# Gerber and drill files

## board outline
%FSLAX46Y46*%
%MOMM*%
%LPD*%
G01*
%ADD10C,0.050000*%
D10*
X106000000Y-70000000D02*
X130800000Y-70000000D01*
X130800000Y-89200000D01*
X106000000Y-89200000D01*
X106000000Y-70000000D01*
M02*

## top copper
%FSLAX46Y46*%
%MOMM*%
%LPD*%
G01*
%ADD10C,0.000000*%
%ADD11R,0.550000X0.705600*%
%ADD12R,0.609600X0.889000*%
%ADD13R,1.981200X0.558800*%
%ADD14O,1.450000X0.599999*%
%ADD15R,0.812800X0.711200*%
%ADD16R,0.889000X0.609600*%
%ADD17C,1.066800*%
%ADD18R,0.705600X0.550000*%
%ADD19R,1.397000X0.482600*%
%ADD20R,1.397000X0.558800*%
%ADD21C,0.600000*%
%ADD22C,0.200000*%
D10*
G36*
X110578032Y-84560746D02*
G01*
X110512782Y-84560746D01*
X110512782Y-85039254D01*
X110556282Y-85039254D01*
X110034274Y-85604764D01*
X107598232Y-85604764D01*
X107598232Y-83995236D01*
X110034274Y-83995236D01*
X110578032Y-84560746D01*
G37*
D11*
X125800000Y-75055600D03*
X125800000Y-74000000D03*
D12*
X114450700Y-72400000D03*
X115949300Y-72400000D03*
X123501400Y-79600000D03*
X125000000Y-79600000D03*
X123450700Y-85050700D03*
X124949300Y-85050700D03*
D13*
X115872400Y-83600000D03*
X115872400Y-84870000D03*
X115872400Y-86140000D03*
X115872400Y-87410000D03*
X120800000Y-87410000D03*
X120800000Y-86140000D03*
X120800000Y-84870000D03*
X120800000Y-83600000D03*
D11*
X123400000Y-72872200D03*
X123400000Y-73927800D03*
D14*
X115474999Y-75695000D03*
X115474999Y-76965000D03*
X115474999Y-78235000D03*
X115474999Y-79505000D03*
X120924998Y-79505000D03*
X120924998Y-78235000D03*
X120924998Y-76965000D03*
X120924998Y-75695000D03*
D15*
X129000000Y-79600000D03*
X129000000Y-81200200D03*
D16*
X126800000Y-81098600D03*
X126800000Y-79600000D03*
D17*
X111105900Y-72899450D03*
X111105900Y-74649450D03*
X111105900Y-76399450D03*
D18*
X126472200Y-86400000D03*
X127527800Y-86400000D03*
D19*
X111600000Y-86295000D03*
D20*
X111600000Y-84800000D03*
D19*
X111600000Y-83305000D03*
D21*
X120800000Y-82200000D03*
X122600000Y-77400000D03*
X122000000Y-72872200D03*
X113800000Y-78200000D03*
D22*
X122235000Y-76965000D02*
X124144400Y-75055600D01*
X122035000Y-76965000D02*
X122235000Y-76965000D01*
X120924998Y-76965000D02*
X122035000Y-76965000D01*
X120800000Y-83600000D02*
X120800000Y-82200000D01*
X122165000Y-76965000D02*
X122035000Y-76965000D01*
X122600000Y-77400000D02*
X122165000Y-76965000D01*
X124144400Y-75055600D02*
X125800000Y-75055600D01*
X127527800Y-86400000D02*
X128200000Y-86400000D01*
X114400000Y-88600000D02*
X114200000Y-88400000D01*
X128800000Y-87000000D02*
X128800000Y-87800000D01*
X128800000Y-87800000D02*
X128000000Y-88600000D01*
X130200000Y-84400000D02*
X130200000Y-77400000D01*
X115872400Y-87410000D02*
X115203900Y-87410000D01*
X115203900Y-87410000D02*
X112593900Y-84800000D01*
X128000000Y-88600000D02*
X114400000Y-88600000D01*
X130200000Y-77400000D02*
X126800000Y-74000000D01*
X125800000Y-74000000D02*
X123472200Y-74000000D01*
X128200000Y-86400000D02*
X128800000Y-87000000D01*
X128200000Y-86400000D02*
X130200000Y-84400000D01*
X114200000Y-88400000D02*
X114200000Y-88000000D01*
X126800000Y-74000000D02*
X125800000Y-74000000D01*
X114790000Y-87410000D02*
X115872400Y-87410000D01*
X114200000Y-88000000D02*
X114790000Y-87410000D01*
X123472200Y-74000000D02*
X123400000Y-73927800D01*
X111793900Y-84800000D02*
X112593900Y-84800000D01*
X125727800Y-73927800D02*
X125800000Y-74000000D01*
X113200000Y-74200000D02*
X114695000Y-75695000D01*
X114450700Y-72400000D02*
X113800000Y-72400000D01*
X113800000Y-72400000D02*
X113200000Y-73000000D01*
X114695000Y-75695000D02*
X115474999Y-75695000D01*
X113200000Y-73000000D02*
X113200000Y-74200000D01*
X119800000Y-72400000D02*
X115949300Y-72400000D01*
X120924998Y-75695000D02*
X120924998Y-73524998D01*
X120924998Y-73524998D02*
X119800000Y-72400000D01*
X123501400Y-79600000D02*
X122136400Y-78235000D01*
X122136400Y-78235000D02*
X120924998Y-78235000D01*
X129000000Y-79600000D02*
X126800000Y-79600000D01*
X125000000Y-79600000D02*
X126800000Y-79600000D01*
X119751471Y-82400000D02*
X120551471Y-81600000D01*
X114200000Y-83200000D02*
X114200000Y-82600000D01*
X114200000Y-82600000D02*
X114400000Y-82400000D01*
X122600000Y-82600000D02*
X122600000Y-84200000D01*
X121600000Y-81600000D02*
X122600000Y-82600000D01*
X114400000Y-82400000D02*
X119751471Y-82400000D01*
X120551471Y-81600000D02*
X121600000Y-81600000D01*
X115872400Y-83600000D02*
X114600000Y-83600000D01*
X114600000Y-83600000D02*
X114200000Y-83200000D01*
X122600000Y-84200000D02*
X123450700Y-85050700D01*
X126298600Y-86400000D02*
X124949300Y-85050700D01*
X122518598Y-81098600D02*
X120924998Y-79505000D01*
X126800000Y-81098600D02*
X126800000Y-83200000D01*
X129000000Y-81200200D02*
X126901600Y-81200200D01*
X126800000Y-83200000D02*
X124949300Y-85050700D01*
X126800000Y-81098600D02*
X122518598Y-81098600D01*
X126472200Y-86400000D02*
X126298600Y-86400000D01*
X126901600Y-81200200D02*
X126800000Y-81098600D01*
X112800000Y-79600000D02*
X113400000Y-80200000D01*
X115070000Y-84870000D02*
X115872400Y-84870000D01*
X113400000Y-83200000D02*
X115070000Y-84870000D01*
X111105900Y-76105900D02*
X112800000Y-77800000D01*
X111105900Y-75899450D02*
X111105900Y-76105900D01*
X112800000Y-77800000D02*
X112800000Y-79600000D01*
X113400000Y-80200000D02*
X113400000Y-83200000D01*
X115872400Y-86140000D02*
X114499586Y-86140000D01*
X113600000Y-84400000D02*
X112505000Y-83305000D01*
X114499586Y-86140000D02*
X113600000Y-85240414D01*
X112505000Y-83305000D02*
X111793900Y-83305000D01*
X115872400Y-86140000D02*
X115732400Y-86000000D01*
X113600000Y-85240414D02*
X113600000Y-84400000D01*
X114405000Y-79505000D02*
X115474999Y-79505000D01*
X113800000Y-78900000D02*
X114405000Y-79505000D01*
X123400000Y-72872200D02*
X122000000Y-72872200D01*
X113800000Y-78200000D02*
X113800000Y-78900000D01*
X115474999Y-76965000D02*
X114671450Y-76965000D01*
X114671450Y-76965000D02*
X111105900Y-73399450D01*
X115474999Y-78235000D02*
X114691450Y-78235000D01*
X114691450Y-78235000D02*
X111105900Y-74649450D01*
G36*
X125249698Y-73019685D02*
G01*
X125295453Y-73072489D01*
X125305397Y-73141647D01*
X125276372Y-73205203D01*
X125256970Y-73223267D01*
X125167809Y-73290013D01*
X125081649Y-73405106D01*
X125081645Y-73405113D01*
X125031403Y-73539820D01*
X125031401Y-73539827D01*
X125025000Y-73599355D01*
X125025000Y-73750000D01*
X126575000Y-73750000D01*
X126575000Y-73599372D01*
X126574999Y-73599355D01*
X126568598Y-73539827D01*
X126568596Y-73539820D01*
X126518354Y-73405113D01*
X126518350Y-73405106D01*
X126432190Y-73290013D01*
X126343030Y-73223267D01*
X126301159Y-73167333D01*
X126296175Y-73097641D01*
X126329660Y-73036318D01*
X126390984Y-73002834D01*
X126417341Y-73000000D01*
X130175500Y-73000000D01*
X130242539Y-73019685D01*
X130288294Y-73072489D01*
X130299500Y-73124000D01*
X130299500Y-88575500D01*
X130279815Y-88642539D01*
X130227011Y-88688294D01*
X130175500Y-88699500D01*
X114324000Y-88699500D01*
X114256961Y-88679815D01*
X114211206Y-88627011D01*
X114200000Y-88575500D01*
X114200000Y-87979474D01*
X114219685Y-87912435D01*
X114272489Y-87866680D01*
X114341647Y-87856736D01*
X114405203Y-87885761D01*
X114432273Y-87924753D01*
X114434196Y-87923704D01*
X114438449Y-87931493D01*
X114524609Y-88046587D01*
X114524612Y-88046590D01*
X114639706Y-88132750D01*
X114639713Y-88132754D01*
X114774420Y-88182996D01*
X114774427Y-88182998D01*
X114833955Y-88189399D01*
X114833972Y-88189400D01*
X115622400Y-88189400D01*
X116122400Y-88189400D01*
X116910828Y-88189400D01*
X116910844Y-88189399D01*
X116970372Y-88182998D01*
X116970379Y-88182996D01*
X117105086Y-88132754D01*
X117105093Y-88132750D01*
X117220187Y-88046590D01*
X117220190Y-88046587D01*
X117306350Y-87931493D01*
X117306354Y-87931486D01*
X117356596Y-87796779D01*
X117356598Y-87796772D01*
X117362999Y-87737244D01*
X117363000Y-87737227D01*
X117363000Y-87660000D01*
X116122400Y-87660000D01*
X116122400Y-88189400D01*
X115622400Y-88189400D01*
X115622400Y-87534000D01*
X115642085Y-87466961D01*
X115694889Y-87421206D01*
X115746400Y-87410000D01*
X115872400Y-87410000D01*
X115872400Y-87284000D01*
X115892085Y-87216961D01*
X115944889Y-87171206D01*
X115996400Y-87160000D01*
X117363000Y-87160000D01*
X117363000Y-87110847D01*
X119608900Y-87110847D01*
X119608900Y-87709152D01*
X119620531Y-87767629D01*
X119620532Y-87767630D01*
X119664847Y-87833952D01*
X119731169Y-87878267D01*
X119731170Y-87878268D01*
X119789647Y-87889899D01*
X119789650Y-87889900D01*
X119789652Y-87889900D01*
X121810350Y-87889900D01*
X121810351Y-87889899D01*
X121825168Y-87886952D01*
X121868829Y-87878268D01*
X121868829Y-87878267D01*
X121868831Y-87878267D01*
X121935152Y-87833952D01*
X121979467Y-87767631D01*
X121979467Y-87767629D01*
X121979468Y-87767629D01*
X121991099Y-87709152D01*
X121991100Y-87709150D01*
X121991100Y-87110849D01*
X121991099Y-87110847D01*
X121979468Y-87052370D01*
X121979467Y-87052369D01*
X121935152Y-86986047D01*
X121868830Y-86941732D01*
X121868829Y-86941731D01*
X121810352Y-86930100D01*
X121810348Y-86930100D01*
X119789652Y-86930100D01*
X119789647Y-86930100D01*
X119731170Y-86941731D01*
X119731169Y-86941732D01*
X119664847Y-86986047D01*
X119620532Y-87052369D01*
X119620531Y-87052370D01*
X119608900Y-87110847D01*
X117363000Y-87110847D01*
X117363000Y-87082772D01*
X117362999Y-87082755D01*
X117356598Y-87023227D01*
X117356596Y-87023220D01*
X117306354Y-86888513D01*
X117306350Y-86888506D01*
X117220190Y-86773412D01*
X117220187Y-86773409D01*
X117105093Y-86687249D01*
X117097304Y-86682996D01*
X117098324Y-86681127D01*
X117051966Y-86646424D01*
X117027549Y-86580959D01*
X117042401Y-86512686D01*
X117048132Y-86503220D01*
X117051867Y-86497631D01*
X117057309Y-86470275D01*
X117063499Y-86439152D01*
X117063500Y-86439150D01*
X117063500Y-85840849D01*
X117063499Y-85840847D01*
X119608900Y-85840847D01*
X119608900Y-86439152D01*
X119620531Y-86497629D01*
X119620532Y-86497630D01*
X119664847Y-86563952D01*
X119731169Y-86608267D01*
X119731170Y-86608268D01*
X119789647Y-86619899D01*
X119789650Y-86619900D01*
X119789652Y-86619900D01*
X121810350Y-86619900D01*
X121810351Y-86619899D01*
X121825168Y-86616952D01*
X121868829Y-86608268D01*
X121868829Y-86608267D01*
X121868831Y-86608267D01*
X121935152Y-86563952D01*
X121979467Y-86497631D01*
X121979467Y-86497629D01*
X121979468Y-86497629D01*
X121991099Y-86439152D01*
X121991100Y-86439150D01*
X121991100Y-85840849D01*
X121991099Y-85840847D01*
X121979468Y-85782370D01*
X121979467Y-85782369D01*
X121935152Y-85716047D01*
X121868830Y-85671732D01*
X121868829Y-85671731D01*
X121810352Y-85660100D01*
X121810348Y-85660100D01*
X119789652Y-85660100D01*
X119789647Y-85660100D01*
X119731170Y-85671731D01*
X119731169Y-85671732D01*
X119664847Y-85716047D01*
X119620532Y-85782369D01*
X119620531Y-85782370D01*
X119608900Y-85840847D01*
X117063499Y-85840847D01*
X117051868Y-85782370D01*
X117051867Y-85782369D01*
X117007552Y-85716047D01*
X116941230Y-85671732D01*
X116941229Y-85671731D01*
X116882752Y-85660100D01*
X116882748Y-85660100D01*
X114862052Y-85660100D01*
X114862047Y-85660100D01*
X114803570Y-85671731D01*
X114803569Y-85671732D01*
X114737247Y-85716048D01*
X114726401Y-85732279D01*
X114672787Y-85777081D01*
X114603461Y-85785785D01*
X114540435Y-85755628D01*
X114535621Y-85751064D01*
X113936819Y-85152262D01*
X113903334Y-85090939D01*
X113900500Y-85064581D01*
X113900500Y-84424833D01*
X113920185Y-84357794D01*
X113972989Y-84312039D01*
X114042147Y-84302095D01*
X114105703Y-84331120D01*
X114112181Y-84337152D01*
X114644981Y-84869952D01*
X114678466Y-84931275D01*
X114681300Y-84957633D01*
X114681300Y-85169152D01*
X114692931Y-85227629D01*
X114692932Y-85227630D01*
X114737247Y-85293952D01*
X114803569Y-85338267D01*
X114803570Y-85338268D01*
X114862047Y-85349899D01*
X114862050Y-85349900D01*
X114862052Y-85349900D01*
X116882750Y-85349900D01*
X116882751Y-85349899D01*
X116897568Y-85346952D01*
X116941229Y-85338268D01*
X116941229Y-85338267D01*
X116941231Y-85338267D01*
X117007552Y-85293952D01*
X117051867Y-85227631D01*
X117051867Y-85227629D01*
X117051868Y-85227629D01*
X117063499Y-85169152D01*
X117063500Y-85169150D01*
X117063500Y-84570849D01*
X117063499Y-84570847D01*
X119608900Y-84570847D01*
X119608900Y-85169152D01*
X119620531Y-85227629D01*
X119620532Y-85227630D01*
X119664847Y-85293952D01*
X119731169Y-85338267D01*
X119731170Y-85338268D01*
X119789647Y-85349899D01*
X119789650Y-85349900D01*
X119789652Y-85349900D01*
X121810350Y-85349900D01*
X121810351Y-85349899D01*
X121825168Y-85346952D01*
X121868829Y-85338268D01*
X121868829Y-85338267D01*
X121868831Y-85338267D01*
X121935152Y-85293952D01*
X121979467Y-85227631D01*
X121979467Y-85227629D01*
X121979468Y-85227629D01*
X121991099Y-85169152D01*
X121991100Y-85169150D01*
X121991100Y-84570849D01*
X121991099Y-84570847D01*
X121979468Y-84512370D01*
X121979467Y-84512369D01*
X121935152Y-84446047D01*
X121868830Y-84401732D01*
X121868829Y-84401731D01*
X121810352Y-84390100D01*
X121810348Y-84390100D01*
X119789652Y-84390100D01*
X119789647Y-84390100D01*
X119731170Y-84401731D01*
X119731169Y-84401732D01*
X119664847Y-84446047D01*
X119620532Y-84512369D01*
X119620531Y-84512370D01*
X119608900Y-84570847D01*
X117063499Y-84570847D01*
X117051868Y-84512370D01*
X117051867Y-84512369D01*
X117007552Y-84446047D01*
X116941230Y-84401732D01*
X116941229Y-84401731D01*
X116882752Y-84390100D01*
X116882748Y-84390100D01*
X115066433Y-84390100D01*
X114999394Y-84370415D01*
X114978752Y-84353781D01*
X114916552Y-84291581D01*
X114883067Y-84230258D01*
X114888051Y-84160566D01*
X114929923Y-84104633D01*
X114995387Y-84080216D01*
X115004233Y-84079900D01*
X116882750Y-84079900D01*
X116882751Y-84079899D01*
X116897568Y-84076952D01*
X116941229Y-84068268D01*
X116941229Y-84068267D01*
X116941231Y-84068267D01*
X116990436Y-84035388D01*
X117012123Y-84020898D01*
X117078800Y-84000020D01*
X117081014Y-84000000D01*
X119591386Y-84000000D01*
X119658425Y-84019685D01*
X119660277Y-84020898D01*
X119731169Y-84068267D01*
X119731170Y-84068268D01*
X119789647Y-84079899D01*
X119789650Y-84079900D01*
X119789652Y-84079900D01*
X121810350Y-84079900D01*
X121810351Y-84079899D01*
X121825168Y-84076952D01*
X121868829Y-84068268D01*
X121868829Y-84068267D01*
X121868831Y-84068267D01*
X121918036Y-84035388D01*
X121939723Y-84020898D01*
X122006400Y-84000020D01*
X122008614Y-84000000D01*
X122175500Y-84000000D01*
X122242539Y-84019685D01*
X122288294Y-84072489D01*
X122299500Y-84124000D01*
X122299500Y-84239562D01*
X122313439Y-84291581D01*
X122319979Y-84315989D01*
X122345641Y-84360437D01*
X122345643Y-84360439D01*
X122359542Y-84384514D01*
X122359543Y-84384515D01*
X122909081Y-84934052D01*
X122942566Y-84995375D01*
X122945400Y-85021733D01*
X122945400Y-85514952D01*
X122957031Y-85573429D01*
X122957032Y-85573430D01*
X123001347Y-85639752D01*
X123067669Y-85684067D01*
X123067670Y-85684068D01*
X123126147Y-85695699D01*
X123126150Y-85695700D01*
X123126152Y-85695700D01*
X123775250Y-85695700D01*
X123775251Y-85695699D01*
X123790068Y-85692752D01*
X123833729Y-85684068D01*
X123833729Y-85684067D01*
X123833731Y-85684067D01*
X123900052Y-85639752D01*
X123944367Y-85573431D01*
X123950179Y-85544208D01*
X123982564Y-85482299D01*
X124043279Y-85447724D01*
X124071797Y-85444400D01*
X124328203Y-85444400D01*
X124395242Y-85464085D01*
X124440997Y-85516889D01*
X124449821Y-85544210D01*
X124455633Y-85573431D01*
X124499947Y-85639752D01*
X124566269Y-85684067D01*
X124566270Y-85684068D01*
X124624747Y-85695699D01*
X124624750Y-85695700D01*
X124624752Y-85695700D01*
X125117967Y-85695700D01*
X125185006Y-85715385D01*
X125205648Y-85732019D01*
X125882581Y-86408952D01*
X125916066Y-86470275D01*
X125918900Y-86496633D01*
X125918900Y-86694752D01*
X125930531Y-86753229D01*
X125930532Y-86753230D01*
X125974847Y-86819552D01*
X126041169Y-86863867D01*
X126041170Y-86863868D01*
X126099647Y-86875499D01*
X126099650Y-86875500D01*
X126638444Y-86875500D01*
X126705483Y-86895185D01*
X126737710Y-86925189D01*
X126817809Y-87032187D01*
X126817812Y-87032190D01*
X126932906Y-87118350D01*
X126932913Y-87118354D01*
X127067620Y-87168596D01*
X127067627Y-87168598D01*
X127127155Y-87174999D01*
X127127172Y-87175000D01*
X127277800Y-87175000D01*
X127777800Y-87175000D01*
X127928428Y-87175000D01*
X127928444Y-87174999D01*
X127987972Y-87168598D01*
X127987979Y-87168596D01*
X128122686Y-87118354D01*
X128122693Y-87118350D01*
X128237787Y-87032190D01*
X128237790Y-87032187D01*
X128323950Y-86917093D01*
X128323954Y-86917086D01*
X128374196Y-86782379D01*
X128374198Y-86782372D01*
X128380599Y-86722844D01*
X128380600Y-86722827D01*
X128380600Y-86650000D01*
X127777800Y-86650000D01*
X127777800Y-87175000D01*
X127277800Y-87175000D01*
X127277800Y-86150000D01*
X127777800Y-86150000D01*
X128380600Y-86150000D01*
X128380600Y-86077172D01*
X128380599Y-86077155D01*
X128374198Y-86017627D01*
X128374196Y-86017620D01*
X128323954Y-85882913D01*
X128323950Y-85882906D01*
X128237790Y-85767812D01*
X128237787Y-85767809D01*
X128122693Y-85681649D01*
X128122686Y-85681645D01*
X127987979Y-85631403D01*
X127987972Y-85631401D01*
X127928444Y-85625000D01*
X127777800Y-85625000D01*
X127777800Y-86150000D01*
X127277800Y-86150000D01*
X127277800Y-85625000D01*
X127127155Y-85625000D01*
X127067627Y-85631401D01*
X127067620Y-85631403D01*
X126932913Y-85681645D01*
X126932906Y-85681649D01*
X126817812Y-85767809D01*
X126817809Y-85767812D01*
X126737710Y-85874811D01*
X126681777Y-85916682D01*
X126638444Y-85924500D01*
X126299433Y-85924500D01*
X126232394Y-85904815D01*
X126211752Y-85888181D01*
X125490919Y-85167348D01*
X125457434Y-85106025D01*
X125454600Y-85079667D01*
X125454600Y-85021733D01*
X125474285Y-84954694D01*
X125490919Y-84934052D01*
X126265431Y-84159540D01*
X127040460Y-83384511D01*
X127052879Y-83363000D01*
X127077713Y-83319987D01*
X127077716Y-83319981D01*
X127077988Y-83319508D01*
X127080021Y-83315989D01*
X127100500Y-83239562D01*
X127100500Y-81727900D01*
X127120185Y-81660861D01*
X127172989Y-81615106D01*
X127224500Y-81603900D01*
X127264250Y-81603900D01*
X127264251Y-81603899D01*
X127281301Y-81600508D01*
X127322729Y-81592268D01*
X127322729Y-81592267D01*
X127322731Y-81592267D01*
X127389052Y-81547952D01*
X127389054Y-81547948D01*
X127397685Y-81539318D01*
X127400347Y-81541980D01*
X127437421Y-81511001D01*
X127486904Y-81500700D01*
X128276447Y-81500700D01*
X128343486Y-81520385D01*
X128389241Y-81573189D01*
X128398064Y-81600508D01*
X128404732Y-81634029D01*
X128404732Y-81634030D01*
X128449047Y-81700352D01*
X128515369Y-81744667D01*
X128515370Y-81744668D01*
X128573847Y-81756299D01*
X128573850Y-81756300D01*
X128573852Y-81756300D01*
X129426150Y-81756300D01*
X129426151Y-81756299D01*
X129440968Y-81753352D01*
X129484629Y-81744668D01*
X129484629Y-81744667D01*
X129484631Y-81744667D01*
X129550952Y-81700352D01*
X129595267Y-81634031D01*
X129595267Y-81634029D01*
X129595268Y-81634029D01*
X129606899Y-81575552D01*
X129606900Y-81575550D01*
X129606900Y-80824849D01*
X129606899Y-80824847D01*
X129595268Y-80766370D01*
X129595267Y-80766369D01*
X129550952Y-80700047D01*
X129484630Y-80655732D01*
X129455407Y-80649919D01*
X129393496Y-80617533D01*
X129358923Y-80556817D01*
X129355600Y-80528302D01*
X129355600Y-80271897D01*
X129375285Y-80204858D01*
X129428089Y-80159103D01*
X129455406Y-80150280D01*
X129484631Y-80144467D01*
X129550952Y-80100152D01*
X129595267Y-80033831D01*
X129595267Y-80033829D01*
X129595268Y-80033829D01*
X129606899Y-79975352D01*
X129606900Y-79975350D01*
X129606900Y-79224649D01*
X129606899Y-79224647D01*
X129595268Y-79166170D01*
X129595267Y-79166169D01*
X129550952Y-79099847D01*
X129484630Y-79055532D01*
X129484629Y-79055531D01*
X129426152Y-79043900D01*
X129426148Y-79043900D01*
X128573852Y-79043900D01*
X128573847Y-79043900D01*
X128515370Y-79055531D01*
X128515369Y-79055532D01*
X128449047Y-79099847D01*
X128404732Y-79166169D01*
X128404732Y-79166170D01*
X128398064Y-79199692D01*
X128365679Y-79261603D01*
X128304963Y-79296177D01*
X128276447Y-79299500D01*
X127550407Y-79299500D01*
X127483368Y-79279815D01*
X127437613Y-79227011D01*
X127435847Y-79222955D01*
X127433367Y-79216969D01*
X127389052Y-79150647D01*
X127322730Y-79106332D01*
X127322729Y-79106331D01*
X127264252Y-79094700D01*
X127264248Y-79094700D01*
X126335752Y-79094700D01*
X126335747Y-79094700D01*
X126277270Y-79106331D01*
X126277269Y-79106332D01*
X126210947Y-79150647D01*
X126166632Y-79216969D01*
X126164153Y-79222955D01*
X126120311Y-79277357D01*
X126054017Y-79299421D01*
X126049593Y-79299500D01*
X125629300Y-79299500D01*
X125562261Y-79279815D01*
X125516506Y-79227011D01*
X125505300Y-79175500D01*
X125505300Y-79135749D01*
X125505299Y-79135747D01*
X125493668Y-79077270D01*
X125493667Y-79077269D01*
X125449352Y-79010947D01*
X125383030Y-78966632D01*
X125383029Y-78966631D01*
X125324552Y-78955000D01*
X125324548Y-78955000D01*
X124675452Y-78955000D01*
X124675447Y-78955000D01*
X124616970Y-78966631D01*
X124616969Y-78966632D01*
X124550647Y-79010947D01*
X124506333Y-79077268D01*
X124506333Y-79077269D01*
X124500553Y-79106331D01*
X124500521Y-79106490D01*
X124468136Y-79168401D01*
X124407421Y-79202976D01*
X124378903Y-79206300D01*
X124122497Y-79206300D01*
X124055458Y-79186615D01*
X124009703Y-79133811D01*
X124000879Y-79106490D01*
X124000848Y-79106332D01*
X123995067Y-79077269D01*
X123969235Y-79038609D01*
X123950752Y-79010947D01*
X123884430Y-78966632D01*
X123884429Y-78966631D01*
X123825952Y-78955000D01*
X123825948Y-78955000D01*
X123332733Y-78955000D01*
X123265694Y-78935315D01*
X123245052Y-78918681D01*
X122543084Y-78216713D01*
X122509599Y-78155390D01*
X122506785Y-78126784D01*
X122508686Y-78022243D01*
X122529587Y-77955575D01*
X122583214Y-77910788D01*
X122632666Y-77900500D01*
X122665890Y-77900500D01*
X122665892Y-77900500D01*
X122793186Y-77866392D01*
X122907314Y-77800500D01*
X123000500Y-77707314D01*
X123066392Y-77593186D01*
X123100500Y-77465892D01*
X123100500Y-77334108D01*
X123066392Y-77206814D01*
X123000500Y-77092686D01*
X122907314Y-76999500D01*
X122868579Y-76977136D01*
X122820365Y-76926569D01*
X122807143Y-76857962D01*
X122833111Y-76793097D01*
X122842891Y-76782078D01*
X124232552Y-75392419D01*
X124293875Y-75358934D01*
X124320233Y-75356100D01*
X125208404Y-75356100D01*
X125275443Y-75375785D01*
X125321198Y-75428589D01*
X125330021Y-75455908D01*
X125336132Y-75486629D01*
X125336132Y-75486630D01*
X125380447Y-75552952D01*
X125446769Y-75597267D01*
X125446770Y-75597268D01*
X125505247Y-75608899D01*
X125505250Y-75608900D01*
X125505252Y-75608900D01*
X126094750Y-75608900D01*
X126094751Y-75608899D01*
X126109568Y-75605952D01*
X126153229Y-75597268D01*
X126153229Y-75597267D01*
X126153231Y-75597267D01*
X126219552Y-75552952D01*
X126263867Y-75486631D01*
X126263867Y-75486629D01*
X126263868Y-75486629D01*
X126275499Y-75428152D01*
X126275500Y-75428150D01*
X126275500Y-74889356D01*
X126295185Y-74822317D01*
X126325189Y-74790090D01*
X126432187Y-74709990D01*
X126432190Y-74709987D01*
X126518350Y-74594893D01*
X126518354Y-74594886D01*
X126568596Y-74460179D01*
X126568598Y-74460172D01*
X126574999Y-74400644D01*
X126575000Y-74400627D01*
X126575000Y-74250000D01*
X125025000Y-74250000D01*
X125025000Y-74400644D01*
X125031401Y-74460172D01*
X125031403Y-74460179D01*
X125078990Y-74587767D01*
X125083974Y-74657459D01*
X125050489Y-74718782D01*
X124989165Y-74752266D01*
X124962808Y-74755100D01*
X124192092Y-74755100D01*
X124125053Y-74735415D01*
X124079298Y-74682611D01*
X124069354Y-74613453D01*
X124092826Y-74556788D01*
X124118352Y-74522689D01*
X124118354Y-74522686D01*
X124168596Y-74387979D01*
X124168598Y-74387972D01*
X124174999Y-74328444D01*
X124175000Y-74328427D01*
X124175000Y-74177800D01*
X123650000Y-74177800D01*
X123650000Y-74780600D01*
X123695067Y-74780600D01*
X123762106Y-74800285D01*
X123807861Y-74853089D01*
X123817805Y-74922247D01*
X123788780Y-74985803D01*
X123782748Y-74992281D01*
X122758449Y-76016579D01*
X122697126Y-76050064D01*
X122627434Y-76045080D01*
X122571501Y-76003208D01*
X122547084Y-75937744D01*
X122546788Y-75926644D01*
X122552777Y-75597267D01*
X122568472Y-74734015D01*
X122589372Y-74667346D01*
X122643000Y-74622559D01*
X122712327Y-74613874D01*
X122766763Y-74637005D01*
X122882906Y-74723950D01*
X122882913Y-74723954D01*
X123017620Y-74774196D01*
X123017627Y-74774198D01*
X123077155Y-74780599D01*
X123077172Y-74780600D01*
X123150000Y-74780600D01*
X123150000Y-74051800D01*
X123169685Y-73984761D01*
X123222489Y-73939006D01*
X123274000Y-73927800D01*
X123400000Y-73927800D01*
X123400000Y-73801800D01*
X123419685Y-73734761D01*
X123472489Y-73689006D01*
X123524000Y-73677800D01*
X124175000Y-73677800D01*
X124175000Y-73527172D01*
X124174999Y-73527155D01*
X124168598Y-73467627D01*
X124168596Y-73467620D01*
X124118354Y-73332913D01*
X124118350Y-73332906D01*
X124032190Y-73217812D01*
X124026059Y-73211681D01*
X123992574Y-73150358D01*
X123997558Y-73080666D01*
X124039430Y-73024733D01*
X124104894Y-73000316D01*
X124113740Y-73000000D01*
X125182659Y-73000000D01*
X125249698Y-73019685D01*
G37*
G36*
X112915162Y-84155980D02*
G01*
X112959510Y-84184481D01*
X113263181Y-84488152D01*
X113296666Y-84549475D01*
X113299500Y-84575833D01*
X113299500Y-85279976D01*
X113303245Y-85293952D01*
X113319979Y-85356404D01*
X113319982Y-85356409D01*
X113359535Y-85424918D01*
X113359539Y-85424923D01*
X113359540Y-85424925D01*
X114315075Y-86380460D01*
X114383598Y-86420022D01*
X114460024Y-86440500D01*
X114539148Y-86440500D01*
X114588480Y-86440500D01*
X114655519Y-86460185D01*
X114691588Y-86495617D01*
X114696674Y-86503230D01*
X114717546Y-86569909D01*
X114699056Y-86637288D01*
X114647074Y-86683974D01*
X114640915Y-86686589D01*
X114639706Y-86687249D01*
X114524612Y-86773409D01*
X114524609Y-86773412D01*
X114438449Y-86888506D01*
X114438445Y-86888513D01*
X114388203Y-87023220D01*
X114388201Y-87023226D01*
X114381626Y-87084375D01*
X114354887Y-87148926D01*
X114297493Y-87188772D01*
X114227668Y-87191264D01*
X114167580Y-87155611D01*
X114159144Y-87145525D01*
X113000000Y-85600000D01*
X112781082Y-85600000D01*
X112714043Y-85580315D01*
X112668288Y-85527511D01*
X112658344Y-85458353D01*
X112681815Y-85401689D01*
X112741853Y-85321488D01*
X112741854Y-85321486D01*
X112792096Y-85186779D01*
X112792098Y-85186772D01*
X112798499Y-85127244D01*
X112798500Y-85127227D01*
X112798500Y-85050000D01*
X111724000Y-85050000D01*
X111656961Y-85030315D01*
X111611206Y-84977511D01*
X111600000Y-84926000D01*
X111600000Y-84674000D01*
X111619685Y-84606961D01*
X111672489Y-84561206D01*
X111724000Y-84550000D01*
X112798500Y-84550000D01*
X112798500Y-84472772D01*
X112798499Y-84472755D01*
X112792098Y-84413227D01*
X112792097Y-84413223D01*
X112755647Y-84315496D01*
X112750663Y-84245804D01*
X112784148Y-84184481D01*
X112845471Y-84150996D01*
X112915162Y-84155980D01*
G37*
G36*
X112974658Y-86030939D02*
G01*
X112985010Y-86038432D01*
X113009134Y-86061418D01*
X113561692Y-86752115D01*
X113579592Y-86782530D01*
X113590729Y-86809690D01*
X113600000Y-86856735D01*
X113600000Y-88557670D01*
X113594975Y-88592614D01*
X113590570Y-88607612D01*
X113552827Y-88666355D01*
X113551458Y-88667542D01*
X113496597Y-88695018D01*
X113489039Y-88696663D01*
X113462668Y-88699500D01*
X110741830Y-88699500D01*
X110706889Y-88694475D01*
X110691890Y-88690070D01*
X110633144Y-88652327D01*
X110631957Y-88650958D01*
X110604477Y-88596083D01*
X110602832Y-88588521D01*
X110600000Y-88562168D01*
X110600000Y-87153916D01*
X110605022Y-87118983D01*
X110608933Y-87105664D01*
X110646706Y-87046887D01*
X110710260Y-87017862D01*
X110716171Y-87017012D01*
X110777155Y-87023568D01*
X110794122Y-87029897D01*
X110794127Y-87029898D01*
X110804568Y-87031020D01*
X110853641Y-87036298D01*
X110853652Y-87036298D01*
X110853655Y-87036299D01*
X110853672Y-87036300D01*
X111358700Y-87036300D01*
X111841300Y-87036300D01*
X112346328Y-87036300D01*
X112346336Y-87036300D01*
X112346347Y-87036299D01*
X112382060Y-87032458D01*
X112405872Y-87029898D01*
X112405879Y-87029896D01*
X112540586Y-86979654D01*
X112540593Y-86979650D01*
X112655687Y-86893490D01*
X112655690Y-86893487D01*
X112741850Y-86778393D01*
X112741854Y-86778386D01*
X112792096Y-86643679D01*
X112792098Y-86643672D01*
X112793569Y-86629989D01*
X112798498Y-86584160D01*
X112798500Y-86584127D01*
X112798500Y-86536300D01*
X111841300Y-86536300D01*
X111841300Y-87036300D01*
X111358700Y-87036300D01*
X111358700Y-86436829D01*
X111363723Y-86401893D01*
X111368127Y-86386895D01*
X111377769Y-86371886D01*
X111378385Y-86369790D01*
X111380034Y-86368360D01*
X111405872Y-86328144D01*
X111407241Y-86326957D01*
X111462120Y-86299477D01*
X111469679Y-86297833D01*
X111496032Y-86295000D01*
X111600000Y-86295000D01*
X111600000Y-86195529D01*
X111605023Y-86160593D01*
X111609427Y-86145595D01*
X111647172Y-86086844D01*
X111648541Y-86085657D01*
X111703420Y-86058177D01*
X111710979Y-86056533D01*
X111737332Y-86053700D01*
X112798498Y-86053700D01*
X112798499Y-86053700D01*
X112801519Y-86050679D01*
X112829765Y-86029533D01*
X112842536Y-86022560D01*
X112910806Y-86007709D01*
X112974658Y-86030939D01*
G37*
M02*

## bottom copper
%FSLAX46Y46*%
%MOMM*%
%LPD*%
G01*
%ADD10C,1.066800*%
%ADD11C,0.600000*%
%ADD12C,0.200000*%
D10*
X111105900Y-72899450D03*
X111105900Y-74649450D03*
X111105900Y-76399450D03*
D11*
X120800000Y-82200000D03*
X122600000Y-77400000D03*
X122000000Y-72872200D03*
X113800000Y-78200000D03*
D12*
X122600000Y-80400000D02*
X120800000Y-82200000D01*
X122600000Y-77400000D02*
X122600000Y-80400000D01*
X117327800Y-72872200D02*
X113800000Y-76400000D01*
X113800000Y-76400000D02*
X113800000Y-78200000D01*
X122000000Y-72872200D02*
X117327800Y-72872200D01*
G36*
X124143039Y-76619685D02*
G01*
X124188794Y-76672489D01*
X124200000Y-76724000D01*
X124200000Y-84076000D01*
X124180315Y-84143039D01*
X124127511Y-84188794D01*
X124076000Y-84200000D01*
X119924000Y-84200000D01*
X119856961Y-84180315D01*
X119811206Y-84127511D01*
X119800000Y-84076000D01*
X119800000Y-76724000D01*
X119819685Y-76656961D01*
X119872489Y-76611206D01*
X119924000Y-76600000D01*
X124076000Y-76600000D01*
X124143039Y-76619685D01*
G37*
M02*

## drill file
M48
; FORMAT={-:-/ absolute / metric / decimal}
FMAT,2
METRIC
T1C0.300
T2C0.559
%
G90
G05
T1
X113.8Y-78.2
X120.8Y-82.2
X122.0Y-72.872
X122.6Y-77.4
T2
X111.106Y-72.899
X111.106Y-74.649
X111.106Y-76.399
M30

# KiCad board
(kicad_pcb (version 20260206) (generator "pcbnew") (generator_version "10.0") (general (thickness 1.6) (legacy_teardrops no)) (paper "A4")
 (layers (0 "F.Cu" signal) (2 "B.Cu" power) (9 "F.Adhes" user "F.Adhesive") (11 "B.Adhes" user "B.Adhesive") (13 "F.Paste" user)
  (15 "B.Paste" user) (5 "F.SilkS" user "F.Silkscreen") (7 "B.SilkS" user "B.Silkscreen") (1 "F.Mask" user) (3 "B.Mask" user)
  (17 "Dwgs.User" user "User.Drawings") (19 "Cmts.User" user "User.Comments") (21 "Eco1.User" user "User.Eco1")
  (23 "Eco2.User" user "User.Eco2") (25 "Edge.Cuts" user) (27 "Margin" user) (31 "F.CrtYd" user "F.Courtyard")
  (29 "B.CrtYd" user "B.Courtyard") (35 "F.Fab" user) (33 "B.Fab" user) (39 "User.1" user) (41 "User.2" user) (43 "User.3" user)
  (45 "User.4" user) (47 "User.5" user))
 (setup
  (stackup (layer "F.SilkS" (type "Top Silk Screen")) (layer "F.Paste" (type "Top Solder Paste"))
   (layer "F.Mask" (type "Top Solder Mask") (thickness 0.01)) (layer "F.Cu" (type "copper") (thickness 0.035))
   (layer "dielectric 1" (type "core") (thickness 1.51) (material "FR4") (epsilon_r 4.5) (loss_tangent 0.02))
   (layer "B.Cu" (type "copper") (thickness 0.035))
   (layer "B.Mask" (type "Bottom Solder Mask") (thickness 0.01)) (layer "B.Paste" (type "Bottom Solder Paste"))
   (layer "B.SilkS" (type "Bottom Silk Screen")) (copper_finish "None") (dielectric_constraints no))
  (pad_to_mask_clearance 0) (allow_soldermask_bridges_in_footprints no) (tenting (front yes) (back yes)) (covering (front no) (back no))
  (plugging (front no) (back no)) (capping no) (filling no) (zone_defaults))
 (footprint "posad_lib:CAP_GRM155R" (layer "F.Cu") (at 125.8 74.5278 90)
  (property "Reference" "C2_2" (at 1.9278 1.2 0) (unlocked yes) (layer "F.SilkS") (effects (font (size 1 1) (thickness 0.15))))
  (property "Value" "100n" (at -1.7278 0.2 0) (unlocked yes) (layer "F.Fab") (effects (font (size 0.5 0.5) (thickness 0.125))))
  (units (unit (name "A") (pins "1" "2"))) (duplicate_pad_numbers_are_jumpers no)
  (pad "1" smd rect (at -0.5278 0 90) (size 0.7056 0.55) (layers "F.Cu" "F.Mask" "F.Paste") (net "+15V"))
  (pad "2" smd rect (at 0.5278 0 90) (size 0.7056 0.55) (layers "F.Cu" "F.Mask" "F.Paste") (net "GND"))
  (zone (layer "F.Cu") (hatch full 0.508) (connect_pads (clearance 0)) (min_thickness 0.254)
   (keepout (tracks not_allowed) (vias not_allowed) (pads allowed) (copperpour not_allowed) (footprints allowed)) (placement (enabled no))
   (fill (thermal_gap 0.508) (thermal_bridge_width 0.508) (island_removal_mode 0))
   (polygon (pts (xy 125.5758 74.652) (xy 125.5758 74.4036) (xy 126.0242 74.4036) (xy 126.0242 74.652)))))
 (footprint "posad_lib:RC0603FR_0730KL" (layer "F.Cu") (at 115.2 72.4)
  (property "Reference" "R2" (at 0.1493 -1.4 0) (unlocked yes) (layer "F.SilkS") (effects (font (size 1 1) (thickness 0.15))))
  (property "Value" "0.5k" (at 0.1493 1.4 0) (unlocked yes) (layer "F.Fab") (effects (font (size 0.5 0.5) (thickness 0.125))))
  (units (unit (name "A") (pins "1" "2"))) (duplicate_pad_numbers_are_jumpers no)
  (pad "1" smd rect (at -0.7493 0) (size 0.6096 0.889) (layers "F.Cu" "F.Mask" "F.Paste") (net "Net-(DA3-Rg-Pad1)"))
  (pad "2" smd rect (at 0.7493 0) (size 0.6096 0.889) (layers "F.Cu" "F.Mask" "F.Paste") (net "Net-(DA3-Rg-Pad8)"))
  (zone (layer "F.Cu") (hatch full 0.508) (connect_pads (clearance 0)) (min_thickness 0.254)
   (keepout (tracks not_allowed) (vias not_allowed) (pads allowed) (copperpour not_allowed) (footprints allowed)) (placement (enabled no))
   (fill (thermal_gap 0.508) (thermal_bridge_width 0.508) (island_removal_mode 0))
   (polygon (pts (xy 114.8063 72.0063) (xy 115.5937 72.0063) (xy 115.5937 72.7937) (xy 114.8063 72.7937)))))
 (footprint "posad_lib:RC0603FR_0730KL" (layer "F.Cu") (at 124.2507 79.6)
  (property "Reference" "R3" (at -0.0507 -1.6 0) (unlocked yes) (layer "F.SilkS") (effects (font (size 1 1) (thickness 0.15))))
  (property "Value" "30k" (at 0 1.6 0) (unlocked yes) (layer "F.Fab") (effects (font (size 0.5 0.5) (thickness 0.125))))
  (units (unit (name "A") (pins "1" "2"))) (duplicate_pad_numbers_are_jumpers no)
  (pad "1" smd rect (at -0.7493 0) (size 0.6096 0.889) (layers "F.Cu" "F.Mask" "F.Paste") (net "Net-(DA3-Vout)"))
  (pad "2" smd rect (at 0.7493 0) (size 0.6096 0.889) (layers "F.Cu" "F.Mask" "F.Paste") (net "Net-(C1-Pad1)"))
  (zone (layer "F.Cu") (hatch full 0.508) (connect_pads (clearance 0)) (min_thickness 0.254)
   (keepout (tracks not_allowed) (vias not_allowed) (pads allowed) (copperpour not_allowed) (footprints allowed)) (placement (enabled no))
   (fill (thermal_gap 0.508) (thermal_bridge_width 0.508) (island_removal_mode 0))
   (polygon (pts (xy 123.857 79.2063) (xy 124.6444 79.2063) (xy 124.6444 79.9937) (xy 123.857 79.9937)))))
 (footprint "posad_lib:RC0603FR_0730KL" (layer "F.Cu") (at 124.2 85.0507)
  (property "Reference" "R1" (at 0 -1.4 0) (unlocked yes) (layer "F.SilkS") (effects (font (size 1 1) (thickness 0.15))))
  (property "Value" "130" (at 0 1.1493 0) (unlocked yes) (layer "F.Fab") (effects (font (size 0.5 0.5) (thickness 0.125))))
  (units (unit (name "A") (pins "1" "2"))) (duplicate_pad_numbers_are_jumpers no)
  (pad "1" smd rect (at -0.7493 0) (size 0.6096 0.889) (layers "F.Cu" "F.Mask" "F.Paste") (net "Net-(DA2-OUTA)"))
  (pad "2" smd rect (at 0.7493 0) (size 0.6096 0.889) (layers "F.Cu" "F.Mask" "F.Paste") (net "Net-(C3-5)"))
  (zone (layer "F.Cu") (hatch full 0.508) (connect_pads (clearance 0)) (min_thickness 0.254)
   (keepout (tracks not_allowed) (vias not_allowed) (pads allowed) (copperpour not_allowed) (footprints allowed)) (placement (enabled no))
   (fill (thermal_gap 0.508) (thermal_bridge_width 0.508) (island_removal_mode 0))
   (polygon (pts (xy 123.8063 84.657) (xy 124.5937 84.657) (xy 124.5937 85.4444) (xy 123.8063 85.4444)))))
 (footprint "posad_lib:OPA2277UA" (layer "F.Cu") (at 118.3362 85.505)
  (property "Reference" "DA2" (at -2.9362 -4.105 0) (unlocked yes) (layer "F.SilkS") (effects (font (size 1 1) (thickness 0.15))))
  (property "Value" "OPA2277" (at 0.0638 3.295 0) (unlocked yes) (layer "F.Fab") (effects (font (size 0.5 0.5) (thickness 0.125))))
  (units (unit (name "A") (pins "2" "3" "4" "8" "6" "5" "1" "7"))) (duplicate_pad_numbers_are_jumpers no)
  (pad "1" smd rect (at -2.4638 -1.905) (size 1.9812 0.5588) (layers "F.Cu" "F.Mask" "F.Paste") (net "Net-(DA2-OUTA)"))
  (pad "2" smd rect (at -2.4638 -0.635) (size 1.9812 0.5588) (layers "F.Cu" "F.Mask" "F.Paste") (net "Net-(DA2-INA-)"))
  (pad "3" smd rect (at -2.4638 0.635) (size 1.9812 0.5588) (layers "F.Cu" "F.Mask" "F.Paste") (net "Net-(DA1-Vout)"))
  (pad "4" smd rect (at -2.4638 1.905) (size 1.9812 0.5588) (layers "F.Cu" "F.Mask" "F.Paste") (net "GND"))
  (pad "5" smd rect (at 2.4638 1.905) (size 1.9812 0.5588) (layers "F.Cu" "F.Mask" "F.Paste") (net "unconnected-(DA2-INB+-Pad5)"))
  (pad "6" smd rect (at 2.4638 0.635) (size 1.9812 0.5588) (layers "F.Cu" "F.Mask" "F.Paste") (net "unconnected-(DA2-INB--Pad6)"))
  (pad "7" smd rect (at 2.4638 -0.635) (size 1.9812 0.5588) (layers "F.Cu" "F.Mask" "F.Paste") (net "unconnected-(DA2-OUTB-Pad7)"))
  (pad "8" smd rect (at 2.4638 -1.905) (size 1.9812 0.5588) (layers "F.Cu" "F.Mask" "F.Paste") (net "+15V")))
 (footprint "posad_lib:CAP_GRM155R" (layer "F.Cu") (at 123.4 73.4 -90)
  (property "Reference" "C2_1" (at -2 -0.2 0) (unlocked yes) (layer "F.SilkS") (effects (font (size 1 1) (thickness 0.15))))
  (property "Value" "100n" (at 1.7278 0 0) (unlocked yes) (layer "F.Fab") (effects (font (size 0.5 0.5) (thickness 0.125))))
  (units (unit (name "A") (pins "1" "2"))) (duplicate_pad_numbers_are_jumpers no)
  (pad "1" smd rect (at -0.5278 0 270) (size 0.7056 0.55) (layers "F.Cu" "F.Mask" "F.Paste") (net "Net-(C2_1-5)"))
  (pad "2" smd rect (at 0.5278 0 270) (size 0.7056 0.55) (layers "F.Cu" "F.Mask" "F.Paste") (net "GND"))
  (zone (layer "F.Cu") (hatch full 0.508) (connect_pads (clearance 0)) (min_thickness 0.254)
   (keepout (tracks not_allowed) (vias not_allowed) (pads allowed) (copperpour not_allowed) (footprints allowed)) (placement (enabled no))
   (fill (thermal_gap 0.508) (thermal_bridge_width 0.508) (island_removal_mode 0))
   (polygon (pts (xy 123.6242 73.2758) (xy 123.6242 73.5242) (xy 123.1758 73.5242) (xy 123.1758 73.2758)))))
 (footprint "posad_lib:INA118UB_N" (layer "F.Cu") (at 118.2 77.6)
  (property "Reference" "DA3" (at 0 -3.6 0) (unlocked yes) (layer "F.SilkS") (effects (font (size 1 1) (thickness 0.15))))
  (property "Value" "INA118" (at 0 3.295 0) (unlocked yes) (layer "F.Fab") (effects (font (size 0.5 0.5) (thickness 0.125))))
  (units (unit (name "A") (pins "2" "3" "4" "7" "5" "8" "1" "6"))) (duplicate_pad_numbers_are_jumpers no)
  (pad "1" smd oval (at -2.725001 -1.905 90) (size 0.599999 1.45) (layers "F.Cu" "F.Mask" "F.Paste") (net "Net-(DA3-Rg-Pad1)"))
  (pad "2" smd oval (at -2.725001 -0.635 90) (size 0.599999 1.45) (layers "F.Cu" "F.Mask" "F.Paste") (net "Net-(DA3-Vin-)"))
  (pad "3" smd oval (at -2.725001 0.635 90) (size 0.599999 1.45) (layers "F.Cu" "F.Mask" "F.Paste") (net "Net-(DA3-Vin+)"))
  (pad "4" smd oval (at -2.725001 1.905 90) (size 0.599999 1.45) (layers "F.Cu" "F.Mask" "F.Paste") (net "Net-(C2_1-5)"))
  (pad "5" smd oval (at 2.724998 1.905 90) (size 0.599999 1.45) (layers "F.Cu" "F.Mask" "F.Paste") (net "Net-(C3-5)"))
  (pad "6" smd oval (at 2.724998 0.635 90) (size 0.599999 1.45) (layers "F.Cu" "F.Mask" "F.Paste") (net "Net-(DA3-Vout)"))
  (pad "7" smd oval (at 2.724998 -0.635 90) (size 0.599999 1.45) (layers "F.Cu" "F.Mask" "F.Paste") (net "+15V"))
  (pad "8" smd oval (at 2.724998 -1.905 90) (size 0.599999 1.45) (layers "F.Cu" "F.Mask" "F.Paste") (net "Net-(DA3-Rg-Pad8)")))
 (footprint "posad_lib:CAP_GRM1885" (layer "F.Cu") (at 129 80.4001 -90)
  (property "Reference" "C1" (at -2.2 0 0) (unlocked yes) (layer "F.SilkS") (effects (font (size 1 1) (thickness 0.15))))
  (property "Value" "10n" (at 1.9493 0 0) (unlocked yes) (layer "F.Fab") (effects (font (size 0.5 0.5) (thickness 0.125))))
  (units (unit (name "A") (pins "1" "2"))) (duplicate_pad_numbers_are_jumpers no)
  (pad "1" smd rect (at -0.8001 0 270) (size 0.7112 0.8128) (layers "F.Cu" "F.Mask" "F.Paste") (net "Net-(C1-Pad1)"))
  (pad "2" smd rect (at 0.8001 0 270) (size 0.7112 0.8128) (layers "F.Cu" "F.Mask" "F.Paste") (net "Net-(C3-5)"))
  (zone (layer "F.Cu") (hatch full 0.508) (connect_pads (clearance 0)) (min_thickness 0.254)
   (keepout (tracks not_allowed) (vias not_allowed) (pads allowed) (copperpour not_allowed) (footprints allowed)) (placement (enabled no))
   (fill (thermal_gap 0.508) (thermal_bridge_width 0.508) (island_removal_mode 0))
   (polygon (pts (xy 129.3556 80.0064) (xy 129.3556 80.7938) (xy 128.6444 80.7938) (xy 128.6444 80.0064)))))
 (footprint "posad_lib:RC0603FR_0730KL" (layer "F.Cu") (at 126.8 80.3493 90)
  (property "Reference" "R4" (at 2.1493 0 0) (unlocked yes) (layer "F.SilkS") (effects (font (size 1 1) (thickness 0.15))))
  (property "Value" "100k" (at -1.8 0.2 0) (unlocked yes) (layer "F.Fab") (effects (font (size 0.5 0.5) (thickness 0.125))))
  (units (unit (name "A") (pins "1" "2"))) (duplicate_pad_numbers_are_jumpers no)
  (pad "1" smd rect (at -0.7493 0 90) (size 0.6096 0.889) (layers "F.Cu" "F.Mask" "F.Paste") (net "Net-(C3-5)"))
  (pad "2" smd rect (at 0.7493 0 90) (size 0.6096 0.889) (layers "F.Cu" "F.Mask" "F.Paste") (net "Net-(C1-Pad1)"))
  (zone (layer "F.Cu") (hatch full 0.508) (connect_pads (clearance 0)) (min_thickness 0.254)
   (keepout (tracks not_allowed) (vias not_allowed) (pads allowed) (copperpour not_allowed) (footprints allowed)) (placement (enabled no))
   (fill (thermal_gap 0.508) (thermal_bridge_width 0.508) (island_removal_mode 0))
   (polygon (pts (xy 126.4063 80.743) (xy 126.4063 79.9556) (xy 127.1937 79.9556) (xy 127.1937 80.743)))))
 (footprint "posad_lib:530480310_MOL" (layer "F.Cu") (at 111.1059 73.39945 -90)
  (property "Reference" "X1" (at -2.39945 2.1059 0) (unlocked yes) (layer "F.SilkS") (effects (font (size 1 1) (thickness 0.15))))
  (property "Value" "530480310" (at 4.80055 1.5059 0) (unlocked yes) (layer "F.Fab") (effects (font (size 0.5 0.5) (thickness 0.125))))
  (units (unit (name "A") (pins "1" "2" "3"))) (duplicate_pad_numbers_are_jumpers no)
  (pad "1" thru_hole circle (at -0.5 0 270) (size 1.0668 1.0668) (drill 0.5588) (layers "*.Cu" "*.Mask") (remove_unused_layers no)
   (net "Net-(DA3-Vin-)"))
  (pad "2" thru_hole circle (at 1.25 0 270) (size 1.0668 1.0668) (drill 0.5588) (layers "*.Cu" "*.Mask") (remove_unused_layers no)
   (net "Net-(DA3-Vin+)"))
  (pad "3" thru_hole circle (at 3 0 270) (size 1.0668 1.0668) (drill 0.5588) (layers "*.Cu" "*.Mask") (remove_unused_layers no)
   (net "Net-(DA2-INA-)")))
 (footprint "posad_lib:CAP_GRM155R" (layer "F.Cu") (at 127 86.4)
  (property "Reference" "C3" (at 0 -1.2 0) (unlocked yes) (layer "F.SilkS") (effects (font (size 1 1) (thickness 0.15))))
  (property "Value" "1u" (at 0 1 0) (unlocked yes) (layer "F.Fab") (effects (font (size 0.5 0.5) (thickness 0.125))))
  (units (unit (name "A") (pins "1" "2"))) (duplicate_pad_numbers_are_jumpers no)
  (pad "1" smd rect (at -0.5278 0) (size 0.7056 0.55) (layers "F.Cu" "F.Mask" "F.Paste") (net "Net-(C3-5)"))
  (pad "2" smd rect (at 0.5278 0) (size 0.7056 0.55) (layers "F.Cu" "F.Mask" "F.Paste") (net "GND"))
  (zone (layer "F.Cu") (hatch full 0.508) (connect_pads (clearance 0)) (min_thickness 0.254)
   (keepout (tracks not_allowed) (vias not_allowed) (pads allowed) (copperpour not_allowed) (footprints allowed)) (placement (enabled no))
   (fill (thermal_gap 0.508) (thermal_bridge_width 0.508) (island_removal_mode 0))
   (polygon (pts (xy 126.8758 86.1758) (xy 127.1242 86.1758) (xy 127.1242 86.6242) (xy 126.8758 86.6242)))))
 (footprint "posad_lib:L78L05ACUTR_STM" (layer "F.Cu") (at 109.6061 84.8 90)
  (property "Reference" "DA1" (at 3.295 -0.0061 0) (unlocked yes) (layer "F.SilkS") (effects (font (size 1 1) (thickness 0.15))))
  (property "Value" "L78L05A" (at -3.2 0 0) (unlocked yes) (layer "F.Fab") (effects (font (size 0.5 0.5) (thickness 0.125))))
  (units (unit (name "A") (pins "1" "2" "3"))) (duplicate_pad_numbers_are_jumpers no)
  (fp_poly
   (pts (xy -0.239254 0.906682) (xy -0.239254 0.950182) (xy -0.804764 0.428174) (xy -0.804764 -2.007868) (xy 0.804764 -2.007868)
    (xy 0.804764 0.428174) (xy 0.239254 0.971932) (xy 0.239254 0.906682))
   (stroke (width 0) (type solid)) (fill yes) (layer "F.Cu"))
  (pad "1" smd rect (at -1.495 1.9939 90) (size 0.4826 1.397) (layers "F.Cu" "F.Mask" "F.Paste") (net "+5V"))
  (pad "2" smd rect (at 0 1.9939 90) (size 0.5588 1.397) (layers "F.Cu" "F.Mask" "F.Paste") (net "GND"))
  (pad "3" smd rect (at 1.495 1.9939 90) (size 0.4826 1.397) (layers "F.Cu" "F.Mask" "F.Paste") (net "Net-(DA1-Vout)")))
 (gr_rect (start 106 70) (end 130.8 89.2) (stroke (width 0.05) (type default)) (fill no) (layer "Edge.Cuts"))
 (segment (start 122.235 76.965) (end 124.1444 75.0556) (width 0.2) (layer "F.Cu") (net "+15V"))
 (segment (start 122.035 76.965) (end 122.235 76.965) (width 0.2) (layer "F.Cu") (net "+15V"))
 (segment (start 120.924998 76.965) (end 122.035 76.965) (width 0.2) (layer "F.Cu") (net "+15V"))
 (segment (start 120.8 83.6) (end 120.8 82.2) (width 0.2) (layer "F.Cu") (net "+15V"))
 (segment (start 122.165 76.965) (end 122.035 76.965) (width 0.2) (layer "F.Cu") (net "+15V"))
 (segment (start 122.6 77.4) (end 122.165 76.965) (width 0.2) (layer "F.Cu") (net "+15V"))
 (segment (start 124.1444 75.0556) (end 125.8 75.0556) (width 0.2) (layer "F.Cu") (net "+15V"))
 (via (at 120.8 82.2) (size 0.6) (drill 0.3) (layers "F.Cu" "B.Cu") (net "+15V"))
 (via (at 122.6 77.4) (size 0.6) (drill 0.3) (layers "F.Cu" "B.Cu") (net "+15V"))
 (segment (start 122.6 80.4) (end 120.8 82.2) (width 0.2) (layer "B.Cu") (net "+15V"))
 (segment (start 122.6 77.4) (end 122.6 80.4) (width 0.2) (layer "B.Cu") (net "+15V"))
 (segment (start 127.5278 86.4) (end 128.2 86.4) (width 0.2) (layer "F.Cu") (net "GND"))
 (segment (start 114.4 88.6) (end 114.2 88.4) (width 0.2) (layer "F.Cu") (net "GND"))
 (segment (start 128.8 87) (end 128.8 87.8) (width 0.2) (layer "F.Cu") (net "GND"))
 (segment (start 128.8 87.8) (end 128 88.6) (width 0.2) (layer "F.Cu") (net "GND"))
 (segment (start 130.2 84.4) (end 130.2 77.4) (width 0.2) (layer "F.Cu") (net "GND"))
 (segment (start 115.8724 87.41) (end 115.2039 87.41) (width 0.2) (layer "F.Cu") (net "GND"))
 (segment (start 115.2039 87.41) (end 112.5939 84.8) (width 0.2) (layer "F.Cu") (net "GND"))
 (segment (start 128 88.6) (end 114.4 88.6) (width 0.2) (layer "F.Cu") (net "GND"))
 (segment (start 130.2 77.4) (end 126.8 74) (width 0.2) (layer "F.Cu") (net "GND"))
 (segment (start 125.8 74) (end 123.4722 74) (width 0.2) (layer "F.Cu") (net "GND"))
 (segment (start 128.2 86.4) (end 128.8 87) (width 0.2) (layer "F.Cu") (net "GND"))
 (segment (start 128.2 86.4) (end 130.2 84.4) (width 0.2) (layer "F.Cu") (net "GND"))
 (segment (start 114.2 88.4) (end 114.2 88) (width 0.2) (layer "F.Cu") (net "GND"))
 (segment (start 126.8 74) (end 125.8 74) (width 0.2) (layer "F.Cu") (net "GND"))
 (segment (start 114.79 87.41) (end 115.8724 87.41) (width 0.2) (layer "F.Cu") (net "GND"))
 (segment (start 114.2 88) (end 114.79 87.41) (width 0.2) (layer "F.Cu") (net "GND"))
 (segment (start 123.4722 74) (end 123.4 73.9278) (width 0.2) (layer "F.Cu") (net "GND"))
 (segment (start 111.7939 84.8) (end 112.5939 84.8) (width 0.2) (layer "F.Cu") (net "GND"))
 (segment (start 125.7278 73.9278) (end 125.8 74) (width 0.2) (layer "F.Cu") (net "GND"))
 (segment (start 113.2 74.2) (end 114.695 75.695) (width 0.2) (layer "F.Cu") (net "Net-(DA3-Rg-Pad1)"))
 (segment (start 114.4507 72.4) (end 113.8 72.4) (width 0.2) (layer "F.Cu") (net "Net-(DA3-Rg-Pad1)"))
 (segment (start 113.8 72.4) (end 113.2 73) (width 0.2) (layer "F.Cu") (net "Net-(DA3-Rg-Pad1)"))
 (segment (start 114.695 75.695) (end 115.474999 75.695) (width 0.2) (layer "F.Cu") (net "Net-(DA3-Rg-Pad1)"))
 (segment (start 113.2 73) (end 113.2 74.2) (width 0.2) (layer "F.Cu") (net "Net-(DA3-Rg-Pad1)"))
 (segment (start 119.8 72.4) (end 115.9493 72.4) (width 0.2) (layer "F.Cu") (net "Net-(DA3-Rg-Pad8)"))
 (segment (start 120.924998 75.695) (end 120.924998 73.524998) (width 0.2) (layer "F.Cu") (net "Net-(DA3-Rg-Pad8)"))
 (segment (start 120.924998 73.524998) (end 119.8 72.4) (width 0.2) (layer "F.Cu") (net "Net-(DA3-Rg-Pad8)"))
 (segment (start 123.5014 79.6) (end 122.1364 78.235) (width 0.2) (layer "F.Cu") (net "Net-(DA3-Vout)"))
 (segment (start 122.1364 78.235) (end 120.924998 78.235) (width 0.2) (layer "F.Cu") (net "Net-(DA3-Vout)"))
 (segment (start 129 79.6) (end 126.8 79.6) (width 0.2) (layer "F.Cu") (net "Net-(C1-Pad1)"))
 (segment (start 125 79.6) (end 126.8 79.6) (width 0.2) (layer "F.Cu") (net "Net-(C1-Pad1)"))
 (segment (start 119.751471 82.4) (end 120.551471 81.6) (width 0.2) (layer "F.Cu") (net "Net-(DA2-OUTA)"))
 (segment (start 114.2 83.2) (end 114.2 82.6) (width 0.2) (layer "F.Cu") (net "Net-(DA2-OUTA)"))
 (segment (start 114.2 82.6) (end 114.4 82.4) (width 0.2) (layer "F.Cu") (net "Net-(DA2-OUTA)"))
 (segment (start 122.6 82.6) (end 122.6 84.2) (width 0.2) (layer "F.Cu") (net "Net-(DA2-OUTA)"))
 (segment (start 121.6 81.6) (end 122.6 82.6) (width 0.2) (layer "F.Cu") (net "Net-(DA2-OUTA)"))
 (segment (start 114.4 82.4) (end 119.751471 82.4) (width 0.2) (layer "F.Cu") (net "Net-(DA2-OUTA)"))
 (segment (start 120.551471 81.6) (end 121.6 81.6) (width 0.2) (layer "F.Cu") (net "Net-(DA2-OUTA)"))
 (segment (start 115.8724 83.6) (end 114.6 83.6) (width 0.2) (layer "F.Cu") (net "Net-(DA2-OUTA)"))
 (segment (start 114.6 83.6) (end 114.2 83.2) (width 0.2) (layer "F.Cu") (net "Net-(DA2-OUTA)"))
 (segment (start 122.6 84.2) (end 123.4507 85.0507) (width 0.2) (layer "F.Cu") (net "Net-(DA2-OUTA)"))
 (segment (start 126.2986 86.4) (end 124.9493 85.0507) (width 0.2) (layer "F.Cu") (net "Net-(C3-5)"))
 (segment (start 122.518598 81.0986) (end 120.924998 79.505) (width 0.2) (layer "F.Cu") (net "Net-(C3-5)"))
 (segment (start 126.8 81.0986) (end 126.8 83.2) (width 0.2) (layer "F.Cu") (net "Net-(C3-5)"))
 (segment (start 129 81.2002) (end 126.9016 81.2002) (width 0.2) (layer "F.Cu") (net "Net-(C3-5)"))
 (segment (start 126.8 83.2) (end 124.9493 85.0507) (width 0.2) (layer "F.Cu") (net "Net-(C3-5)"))
 (segment (start 126.8 81.0986) (end 122.518598 81.0986) (width 0.2) (layer "F.Cu") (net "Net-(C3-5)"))
 (segment (start 126.4722 86.4) (end 126.2986 86.4) (width 0.2) (layer "F.Cu") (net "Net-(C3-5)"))
 (segment (start 126.9016 81.2002) (end 126.8 81.0986) (width 0.2) (layer "F.Cu") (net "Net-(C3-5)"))
 (segment (start 112.8 79.6) (end 113.4 80.2) (width 0.2) (layer "F.Cu") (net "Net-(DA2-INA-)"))
 (segment (start 115.07 84.87) (end 115.8724 84.87) (width 0.2) (layer "F.Cu") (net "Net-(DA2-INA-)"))
 (segment (start 113.4 83.2) (end 115.07 84.87) (width 0.2) (layer "F.Cu") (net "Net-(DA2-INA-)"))
 (segment (start 111.1059 76.1059) (end 112.8 77.8) (width 0.2) (layer "F.Cu") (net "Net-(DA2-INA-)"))
 (segment (start 111.1059 75.89945) (end 111.1059 76.1059) (width 0.2) (layer "F.Cu") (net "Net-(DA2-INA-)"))
 (segment (start 112.8 77.8) (end 112.8 79.6) (width 0.2) (layer "F.Cu") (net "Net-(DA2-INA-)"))
 (segment (start 113.4 80.2) (end 113.4 83.2) (width 0.2) (layer "F.Cu") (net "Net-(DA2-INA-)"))
 (segment (start 115.8724 86.14) (end 114.499586 86.14) (width 0.2) (layer "F.Cu") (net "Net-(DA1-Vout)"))
 (segment (start 113.6 84.4) (end 112.505 83.305) (width 0.2) (layer "F.Cu") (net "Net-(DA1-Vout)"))
 (segment (start 114.499586 86.14) (end 113.6 85.240414) (width 0.2) (layer "F.Cu") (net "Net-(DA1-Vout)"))
 (segment (start 112.505 83.305) (end 111.7939 83.305) (width 0.2) (layer "F.Cu") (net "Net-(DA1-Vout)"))
 (segment (start 115.8724 86.14) (end 115.7324 86) (width 0.2) (layer "F.Cu") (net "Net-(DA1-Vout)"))
 (segment (start 113.6 85.240414) (end 113.6 84.4) (width 0.2) (layer "F.Cu") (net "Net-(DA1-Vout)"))
 (segment (start 114.405 79.505) (end 115.474999 79.505) (width 0.2) (layer "F.Cu") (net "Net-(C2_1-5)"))
 (segment (start 113.8 78.9) (end 114.405 79.505) (width 0.2) (layer "F.Cu") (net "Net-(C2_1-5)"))
 (segment (start 123.4 72.8722) (end 122 72.8722) (width 0.2) (layer "F.Cu") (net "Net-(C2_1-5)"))
 (segment (start 113.8 78.2) (end 113.8 78.9) (width 0.2) (layer "F.Cu") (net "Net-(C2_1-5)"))
 (via (at 122 72.8722) (size 0.6) (drill 0.3) (layers "F.Cu" "B.Cu") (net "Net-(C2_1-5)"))
 (via (at 113.8 78.2) (size 0.6) (drill 0.3) (layers "F.Cu" "B.Cu") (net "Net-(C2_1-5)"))
 (segment (start 117.3278 72.8722) (end 113.8 76.4) (width 0.2) (layer "B.Cu") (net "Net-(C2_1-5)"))
 (segment (start 113.8 76.4) (end 113.8 78.2) (width 0.2) (layer "B.Cu") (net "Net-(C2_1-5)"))
 (segment (start 122 72.8722) (end 117.3278 72.8722) (width 0.2) (layer "B.Cu") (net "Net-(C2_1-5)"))
 (segment (start 115.474999 76.965) (end 114.67145 76.965) (width 0.2) (layer "F.Cu") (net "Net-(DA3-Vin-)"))
 (segment (start 114.67145 76.965) (end 111.1059 73.39945) (width 0.2) (layer "F.Cu") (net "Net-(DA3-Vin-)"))
 (segment (start 115.474999 78.235) (end 114.69145 78.235) (width 0.2) (layer "F.Cu") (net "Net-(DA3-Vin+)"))
 (segment (start 114.69145 78.235) (end 111.1059 74.64945) (width 0.2) (layer "F.Cu") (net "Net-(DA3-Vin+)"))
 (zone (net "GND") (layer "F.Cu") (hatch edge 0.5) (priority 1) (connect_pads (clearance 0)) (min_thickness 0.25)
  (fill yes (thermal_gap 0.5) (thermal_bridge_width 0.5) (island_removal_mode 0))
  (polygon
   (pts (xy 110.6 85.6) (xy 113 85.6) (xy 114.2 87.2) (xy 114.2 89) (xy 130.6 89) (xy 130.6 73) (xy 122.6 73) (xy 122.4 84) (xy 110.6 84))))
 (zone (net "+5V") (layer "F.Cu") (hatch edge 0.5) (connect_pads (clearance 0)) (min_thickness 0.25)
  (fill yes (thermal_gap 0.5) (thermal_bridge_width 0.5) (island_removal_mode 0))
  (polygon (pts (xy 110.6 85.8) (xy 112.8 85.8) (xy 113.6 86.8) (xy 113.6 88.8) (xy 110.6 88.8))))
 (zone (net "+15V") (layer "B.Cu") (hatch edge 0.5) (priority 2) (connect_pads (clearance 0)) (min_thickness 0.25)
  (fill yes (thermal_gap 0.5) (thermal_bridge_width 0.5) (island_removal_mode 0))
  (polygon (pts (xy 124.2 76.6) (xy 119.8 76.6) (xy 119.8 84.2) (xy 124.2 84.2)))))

